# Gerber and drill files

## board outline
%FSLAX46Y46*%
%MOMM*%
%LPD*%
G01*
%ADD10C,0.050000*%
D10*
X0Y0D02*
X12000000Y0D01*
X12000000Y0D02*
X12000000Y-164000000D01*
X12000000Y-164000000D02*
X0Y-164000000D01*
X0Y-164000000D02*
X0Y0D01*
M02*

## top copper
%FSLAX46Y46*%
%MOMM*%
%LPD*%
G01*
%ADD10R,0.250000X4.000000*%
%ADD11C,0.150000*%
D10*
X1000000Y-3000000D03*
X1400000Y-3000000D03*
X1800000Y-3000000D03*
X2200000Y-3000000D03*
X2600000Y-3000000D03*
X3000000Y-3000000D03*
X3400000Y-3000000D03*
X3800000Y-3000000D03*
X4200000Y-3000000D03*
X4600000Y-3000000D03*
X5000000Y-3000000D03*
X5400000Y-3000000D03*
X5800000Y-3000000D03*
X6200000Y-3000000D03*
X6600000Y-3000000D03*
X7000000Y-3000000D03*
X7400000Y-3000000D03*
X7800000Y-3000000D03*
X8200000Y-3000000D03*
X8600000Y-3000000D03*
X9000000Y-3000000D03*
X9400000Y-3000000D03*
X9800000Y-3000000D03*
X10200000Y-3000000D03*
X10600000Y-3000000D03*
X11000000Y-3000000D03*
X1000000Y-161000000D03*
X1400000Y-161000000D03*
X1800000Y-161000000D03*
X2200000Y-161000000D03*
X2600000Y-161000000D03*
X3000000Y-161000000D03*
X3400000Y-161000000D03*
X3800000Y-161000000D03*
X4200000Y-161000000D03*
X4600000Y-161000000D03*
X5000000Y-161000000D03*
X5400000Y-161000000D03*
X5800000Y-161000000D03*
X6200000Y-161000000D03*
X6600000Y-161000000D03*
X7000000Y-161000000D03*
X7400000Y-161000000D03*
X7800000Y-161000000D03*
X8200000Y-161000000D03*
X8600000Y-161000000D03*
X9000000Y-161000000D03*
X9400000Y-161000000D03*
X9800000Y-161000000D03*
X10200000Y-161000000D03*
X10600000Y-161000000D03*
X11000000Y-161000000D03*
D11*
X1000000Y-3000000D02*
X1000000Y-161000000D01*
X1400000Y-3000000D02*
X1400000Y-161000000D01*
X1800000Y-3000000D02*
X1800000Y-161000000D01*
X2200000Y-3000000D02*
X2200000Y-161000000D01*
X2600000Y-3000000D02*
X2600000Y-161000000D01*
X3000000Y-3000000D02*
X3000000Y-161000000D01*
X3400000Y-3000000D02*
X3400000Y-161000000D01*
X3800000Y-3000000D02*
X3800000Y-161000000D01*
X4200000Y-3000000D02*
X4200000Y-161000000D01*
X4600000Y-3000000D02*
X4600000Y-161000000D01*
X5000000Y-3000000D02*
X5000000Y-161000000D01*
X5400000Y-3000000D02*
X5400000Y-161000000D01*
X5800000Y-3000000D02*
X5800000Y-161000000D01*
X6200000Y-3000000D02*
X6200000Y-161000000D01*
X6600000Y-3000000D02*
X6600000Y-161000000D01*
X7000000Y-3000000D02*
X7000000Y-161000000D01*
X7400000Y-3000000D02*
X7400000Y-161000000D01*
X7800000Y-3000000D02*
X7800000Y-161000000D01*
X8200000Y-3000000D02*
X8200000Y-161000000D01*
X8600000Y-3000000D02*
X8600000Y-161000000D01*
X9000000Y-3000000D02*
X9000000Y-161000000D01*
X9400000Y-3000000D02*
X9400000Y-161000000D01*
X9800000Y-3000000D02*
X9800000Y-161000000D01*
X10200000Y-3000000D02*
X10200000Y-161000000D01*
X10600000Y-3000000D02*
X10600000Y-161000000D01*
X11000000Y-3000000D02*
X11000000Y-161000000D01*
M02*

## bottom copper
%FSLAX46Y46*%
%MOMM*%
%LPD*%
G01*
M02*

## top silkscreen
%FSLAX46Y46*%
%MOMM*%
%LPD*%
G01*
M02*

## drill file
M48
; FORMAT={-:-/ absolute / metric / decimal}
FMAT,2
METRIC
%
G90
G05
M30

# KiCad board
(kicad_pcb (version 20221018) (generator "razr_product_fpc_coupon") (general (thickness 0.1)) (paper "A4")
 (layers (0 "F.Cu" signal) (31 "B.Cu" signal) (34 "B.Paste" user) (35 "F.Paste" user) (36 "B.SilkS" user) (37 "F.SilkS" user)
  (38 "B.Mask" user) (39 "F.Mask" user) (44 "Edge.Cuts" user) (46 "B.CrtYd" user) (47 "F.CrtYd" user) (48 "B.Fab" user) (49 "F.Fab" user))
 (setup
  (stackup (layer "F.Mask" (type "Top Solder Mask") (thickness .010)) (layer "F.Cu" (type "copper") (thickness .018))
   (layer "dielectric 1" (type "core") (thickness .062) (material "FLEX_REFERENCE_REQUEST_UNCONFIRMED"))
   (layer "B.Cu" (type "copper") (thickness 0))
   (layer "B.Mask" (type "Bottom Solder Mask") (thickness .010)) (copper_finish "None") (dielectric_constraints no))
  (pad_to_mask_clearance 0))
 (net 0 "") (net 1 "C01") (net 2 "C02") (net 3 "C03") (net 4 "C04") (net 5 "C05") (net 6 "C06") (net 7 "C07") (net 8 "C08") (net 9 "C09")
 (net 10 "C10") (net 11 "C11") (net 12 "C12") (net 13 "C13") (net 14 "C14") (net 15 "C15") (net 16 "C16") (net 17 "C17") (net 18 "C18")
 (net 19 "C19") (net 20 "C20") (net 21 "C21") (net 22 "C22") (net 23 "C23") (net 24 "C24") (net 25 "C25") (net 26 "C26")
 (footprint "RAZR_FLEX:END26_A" (layer "F.Cu") (at 0 0)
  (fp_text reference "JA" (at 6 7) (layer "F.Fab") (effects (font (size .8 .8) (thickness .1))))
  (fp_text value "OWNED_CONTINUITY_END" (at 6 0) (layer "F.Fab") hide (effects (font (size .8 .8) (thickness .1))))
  (pad "1" smd rect (at 1.000000 3.000000) (size 0.25 4.0) (layers "F.Cu" "F.Mask") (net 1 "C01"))
  (pad "2" smd rect (at 1.400000 3.000000) (size 0.25 4.0) (layers "F.Cu" "F.Mask") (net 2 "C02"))
  (pad "3" smd rect (at 1.800000 3.000000) (size 0.25 4.0) (layers "F.Cu" "F.Mask") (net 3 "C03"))
  (pad "4" smd rect (at 2.200000 3.000000) (size 0.25 4.0) (layers "F.Cu" "F.Mask") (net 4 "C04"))
  (pad "5" smd rect (at 2.600000 3.000000) (size 0.25 4.0) (layers "F.Cu" "F.Mask") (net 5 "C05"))
  (pad "6" smd rect (at 3.000000 3.000000) (size 0.25 4.0) (layers "F.Cu" "F.Mask") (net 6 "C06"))
  (pad "7" smd rect (at 3.400000 3.000000) (size 0.25 4.0) (layers "F.Cu" "F.Mask") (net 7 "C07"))
  (pad "8" smd rect (at 3.800000 3.000000) (size 0.25 4.0) (layers "F.Cu" "F.Mask") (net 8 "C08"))
  (pad "9" smd rect (at 4.200000 3.000000) (size 0.25 4.0) (layers "F.Cu" "F.Mask") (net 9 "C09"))
  (pad "10" smd rect (at 4.600000 3.000000) (size 0.25 4.0) (layers "F.Cu" "F.Mask") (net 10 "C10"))
  (pad "11" smd rect (at 5.000000 3.000000) (size 0.25 4.0) (layers "F.Cu" "F.Mask") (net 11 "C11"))
  (pad "12" smd rect (at 5.400000 3.000000) (size 0.25 4.0) (layers "F.Cu" "F.Mask") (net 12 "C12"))
  (pad "13" smd rect (at 5.800000 3.000000) (size 0.25 4.0) (layers "F.Cu" "F.Mask") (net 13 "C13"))
  (pad "14" smd rect (at 6.200000 3.000000) (size 0.25 4.0) (layers "F.Cu" "F.Mask") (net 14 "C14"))
  (pad "15" smd rect (at 6.600000 3.000000) (size 0.25 4.0) (layers "F.Cu" "F.Mask") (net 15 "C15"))
  (pad "16" smd rect (at 7.000000 3.000000) (size 0.25 4.0) (layers "F.Cu" "F.Mask") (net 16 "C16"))
  (pad "17" smd rect (at 7.400000 3.000000) (size 0.25 4.0) (layers "F.Cu" "F.Mask") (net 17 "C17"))
  (pad "18" smd rect (at 7.800000 3.000000) (size 0.25 4.0) (layers "F.Cu" "F.Mask") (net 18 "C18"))
  (pad "19" smd rect (at 8.200000 3.000000) (size 0.25 4.0) (layers "F.Cu" "F.Mask") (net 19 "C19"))
  (pad "20" smd rect (at 8.600000 3.000000) (size 0.25 4.0) (layers "F.Cu" "F.Mask") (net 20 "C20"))
  (pad "21" smd rect (at 9.000000 3.000000) (size 0.25 4.0) (layers "F.Cu" "F.Mask") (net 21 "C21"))
  (pad "22" smd rect (at 9.400000 3.000000) (size 0.25 4.0) (layers "F.Cu" "F.Mask") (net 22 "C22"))
  (pad "23" smd rect (at 9.800000 3.000000) (size 0.25 4.0) (layers "F.Cu" "F.Mask") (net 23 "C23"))
  (pad "24" smd rect (at 10.200000 3.000000) (size 0.25 4.0) (layers "F.Cu" "F.Mask") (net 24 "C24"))
  (pad "25" smd rect (at 10.600000 3.000000) (size 0.25 4.0) (layers "F.Cu" "F.Mask") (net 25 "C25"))
  (pad "26" smd rect (at 11.000000 3.000000) (size 0.25 4.0) (layers "F.Cu" "F.Mask") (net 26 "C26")))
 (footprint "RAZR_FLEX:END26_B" (layer "F.Cu") (at 0 0)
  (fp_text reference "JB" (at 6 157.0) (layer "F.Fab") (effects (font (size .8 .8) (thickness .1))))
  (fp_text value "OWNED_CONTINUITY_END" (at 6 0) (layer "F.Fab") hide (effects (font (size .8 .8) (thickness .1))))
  (pad "1" smd rect (at 1.000000 161.000000) (size 0.25 4.0) (layers "F.Cu" "F.Mask") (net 1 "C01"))
  (pad "2" smd rect (at 1.400000 161.000000) (size 0.25 4.0) (layers "F.Cu" "F.Mask") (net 2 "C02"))
  (pad "3" smd rect (at 1.800000 161.000000) (size 0.25 4.0) (layers "F.Cu" "F.Mask") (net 3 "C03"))
  (pad "4" smd rect (at 2.200000 161.000000) (size 0.25 4.0) (layers "F.Cu" "F.Mask") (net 4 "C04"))
  (pad "5" smd rect (at 2.600000 161.000000) (size 0.25 4.0) (layers "F.Cu" "F.Mask") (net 5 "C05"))
  (pad "6" smd rect (at 3.000000 161.000000) (size 0.25 4.0) (layers "F.Cu" "F.Mask") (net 6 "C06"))
  (pad "7" smd rect (at 3.400000 161.000000) (size 0.25 4.0) (layers "F.Cu" "F.Mask") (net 7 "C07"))
  (pad "8" smd rect (at 3.800000 161.000000) (size 0.25 4.0) (layers "F.Cu" "F.Mask") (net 8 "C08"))
  (pad "9" smd rect (at 4.200000 161.000000) (size 0.25 4.0) (layers "F.Cu" "F.Mask") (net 9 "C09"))
  (pad "10" smd rect (at 4.600000 161.000000) (size 0.25 4.0) (layers "F.Cu" "F.Mask") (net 10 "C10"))
  (pad "11" smd rect (at 5.000000 161.000000) (size 0.25 4.0) (layers "F.Cu" "F.Mask") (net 11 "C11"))
  (pad "12" smd rect (at 5.400000 161.000000) (size 0.25 4.0) (layers "F.Cu" "F.Mask") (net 12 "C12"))
  (pad "13" smd rect (at 5.800000 161.000000) (size 0.25 4.0) (layers "F.Cu" "F.Mask") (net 13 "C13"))
  (pad "14" smd rect (at 6.200000 161.000000) (size 0.25 4.0) (layers "F.Cu" "F.Mask") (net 14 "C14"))
  (pad "15" smd rect (at 6.600000 161.000000) (size 0.25 4.0) (layers "F.Cu" "F.Mask") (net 15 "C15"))
  (pad "16" smd rect (at 7.000000 161.000000) (size 0.25 4.0) (layers "F.Cu" "F.Mask") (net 16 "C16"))
  (pad "17" smd rect (at 7.400000 161.000000) (size 0.25 4.0) (layers "F.Cu" "F.Mask") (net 17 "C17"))
  (pad "18" smd rect (at 7.800000 161.000000) (size 0.25 4.0) (layers "F.Cu" "F.Mask") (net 18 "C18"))
  (pad "19" smd rect (at 8.200000 161.000000) (size 0.25 4.0) (layers "F.Cu" "F.Mask") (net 19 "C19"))
  (pad "20" smd rect (at 8.600000 161.000000) (size 0.25 4.0) (layers "F.Cu" "F.Mask") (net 20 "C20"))
  (pad "21" smd rect (at 9.000000 161.000000) (size 0.25 4.0) (layers "F.Cu" "F.Mask") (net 21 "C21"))
  (pad "22" smd rect (at 9.400000 161.000000) (size 0.25 4.0) (layers "F.Cu" "F.Mask") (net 22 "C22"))
  (pad "23" smd rect (at 9.800000 161.000000) (size 0.25 4.0) (layers "F.Cu" "F.Mask") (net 23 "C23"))
  (pad "24" smd rect (at 10.200000 161.000000) (size 0.25 4.0) (layers "F.Cu" "F.Mask") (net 24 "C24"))
  (pad "25" smd rect (at 10.600000 161.000000) (size 0.25 4.0) (layers "F.Cu" "F.Mask") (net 25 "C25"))
  (pad "26" smd rect (at 11.000000 161.000000) (size 0.25 4.0) (layers "F.Cu" "F.Mask") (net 26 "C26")))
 (segment (start 1.000000 3.000000) (end 1.000000 161.000000) (width 0.15) (layer "F.Cu") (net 1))
 (segment (start 1.400000 3.000000) (end 1.400000 161.000000) (width 0.15) (layer "F.Cu") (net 2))
 (segment (start 1.800000 3.000000) (end 1.800000 161.000000) (width 0.15) (layer "F.Cu") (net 3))
 (segment (start 2.200000 3.000000) (end 2.200000 161.000000) (width 0.15) (layer "F.Cu") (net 4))
 (segment (start 2.600000 3.000000) (end 2.600000 161.000000) (width 0.15) (layer "F.Cu") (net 5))
 (segment (start 3.000000 3.000000) (end 3.000000 161.000000) (width 0.15) (layer "F.Cu") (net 6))
 (segment (start 3.400000 3.000000) (end 3.400000 161.000000) (width 0.15) (layer "F.Cu") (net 7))
 (segment (start 3.800000 3.000000) (end 3.800000 161.000000) (width 0.15) (layer "F.Cu") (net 8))
 (segment (start 4.200000 3.000000) (end 4.200000 161.000000) (width 0.15) (layer "F.Cu") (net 9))
 (segment (start 4.600000 3.000000) (end 4.600000 161.000000) (width 0.15) (layer "F.Cu") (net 10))
 (segment (start 5.000000 3.000000) (end 5.000000 161.000000) (width 0.15) (layer "F.Cu") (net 11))
 (segment (start 5.400000 3.000000) (end 5.400000 161.000000) (width 0.15) (layer "F.Cu") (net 12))
 (segment (start 5.800000 3.000000) (end 5.800000 161.000000) (width 0.15) (layer "F.Cu") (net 13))
 (segment (start 6.200000 3.000000) (end 6.200000 161.000000) (width 0.15) (layer "F.Cu") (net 14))
 (segment (start 6.600000 3.000000) (end 6.600000 161.000000) (width 0.15) (layer "F.Cu") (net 15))
 (segment (start 7.000000 3.000000) (end 7.000000 161.000000) (width 0.15) (layer "F.Cu") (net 16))
 (segment (start 7.400000 3.000000) (end 7.400000 161.000000) (width 0.15) (layer "F.Cu") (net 17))
 (segment (start 7.800000 3.000000) (end 7.800000 161.000000) (width 0.15) (layer "F.Cu") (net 18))
 (segment (start 8.200000 3.000000) (end 8.200000 161.000000) (width 0.15) (layer "F.Cu") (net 19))
 (segment (start 8.600000 3.000000) (end 8.600000 161.000000) (width 0.15) (layer "F.Cu") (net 20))
 (segment (start 9.000000 3.000000) (end 9.000000 161.000000) (width 0.15) (layer "F.Cu") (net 21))
 (segment (start 9.400000 3.000000) (end 9.400000 161.000000) (width 0.15) (layer "F.Cu") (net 22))
 (segment (start 9.800000 3.000000) (end 9.800000 161.000000) (width 0.15) (layer "F.Cu") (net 23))
 (segment (start 10.200000 3.000000) (end 10.200000 161.000000) (width 0.15) (layer "F.Cu") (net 24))
 (segment (start 10.600000 3.000000) (end 10.600000 161.000000) (width 0.15) (layer "F.Cu") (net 25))
 (segment (start 11.000000 3.000000) (end 11.000000 161.000000) (width 0.15) (layer "F.Cu") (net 26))
 (gr_line (start 0 0) (end 12.0 0) (layer "Edge.Cuts") (width .05))
 (gr_line (start 12.0 0) (end 12.0 164.0) (layer "Edge.Cuts") (width .05))
 (gr_line (start 12.0 164.0) (end 0 164.0) (layer "Edge.Cuts") (width .05))
 (gr_line (start 0 164.0) (end 0 0) (layer "Edge.Cuts") (width .05)))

